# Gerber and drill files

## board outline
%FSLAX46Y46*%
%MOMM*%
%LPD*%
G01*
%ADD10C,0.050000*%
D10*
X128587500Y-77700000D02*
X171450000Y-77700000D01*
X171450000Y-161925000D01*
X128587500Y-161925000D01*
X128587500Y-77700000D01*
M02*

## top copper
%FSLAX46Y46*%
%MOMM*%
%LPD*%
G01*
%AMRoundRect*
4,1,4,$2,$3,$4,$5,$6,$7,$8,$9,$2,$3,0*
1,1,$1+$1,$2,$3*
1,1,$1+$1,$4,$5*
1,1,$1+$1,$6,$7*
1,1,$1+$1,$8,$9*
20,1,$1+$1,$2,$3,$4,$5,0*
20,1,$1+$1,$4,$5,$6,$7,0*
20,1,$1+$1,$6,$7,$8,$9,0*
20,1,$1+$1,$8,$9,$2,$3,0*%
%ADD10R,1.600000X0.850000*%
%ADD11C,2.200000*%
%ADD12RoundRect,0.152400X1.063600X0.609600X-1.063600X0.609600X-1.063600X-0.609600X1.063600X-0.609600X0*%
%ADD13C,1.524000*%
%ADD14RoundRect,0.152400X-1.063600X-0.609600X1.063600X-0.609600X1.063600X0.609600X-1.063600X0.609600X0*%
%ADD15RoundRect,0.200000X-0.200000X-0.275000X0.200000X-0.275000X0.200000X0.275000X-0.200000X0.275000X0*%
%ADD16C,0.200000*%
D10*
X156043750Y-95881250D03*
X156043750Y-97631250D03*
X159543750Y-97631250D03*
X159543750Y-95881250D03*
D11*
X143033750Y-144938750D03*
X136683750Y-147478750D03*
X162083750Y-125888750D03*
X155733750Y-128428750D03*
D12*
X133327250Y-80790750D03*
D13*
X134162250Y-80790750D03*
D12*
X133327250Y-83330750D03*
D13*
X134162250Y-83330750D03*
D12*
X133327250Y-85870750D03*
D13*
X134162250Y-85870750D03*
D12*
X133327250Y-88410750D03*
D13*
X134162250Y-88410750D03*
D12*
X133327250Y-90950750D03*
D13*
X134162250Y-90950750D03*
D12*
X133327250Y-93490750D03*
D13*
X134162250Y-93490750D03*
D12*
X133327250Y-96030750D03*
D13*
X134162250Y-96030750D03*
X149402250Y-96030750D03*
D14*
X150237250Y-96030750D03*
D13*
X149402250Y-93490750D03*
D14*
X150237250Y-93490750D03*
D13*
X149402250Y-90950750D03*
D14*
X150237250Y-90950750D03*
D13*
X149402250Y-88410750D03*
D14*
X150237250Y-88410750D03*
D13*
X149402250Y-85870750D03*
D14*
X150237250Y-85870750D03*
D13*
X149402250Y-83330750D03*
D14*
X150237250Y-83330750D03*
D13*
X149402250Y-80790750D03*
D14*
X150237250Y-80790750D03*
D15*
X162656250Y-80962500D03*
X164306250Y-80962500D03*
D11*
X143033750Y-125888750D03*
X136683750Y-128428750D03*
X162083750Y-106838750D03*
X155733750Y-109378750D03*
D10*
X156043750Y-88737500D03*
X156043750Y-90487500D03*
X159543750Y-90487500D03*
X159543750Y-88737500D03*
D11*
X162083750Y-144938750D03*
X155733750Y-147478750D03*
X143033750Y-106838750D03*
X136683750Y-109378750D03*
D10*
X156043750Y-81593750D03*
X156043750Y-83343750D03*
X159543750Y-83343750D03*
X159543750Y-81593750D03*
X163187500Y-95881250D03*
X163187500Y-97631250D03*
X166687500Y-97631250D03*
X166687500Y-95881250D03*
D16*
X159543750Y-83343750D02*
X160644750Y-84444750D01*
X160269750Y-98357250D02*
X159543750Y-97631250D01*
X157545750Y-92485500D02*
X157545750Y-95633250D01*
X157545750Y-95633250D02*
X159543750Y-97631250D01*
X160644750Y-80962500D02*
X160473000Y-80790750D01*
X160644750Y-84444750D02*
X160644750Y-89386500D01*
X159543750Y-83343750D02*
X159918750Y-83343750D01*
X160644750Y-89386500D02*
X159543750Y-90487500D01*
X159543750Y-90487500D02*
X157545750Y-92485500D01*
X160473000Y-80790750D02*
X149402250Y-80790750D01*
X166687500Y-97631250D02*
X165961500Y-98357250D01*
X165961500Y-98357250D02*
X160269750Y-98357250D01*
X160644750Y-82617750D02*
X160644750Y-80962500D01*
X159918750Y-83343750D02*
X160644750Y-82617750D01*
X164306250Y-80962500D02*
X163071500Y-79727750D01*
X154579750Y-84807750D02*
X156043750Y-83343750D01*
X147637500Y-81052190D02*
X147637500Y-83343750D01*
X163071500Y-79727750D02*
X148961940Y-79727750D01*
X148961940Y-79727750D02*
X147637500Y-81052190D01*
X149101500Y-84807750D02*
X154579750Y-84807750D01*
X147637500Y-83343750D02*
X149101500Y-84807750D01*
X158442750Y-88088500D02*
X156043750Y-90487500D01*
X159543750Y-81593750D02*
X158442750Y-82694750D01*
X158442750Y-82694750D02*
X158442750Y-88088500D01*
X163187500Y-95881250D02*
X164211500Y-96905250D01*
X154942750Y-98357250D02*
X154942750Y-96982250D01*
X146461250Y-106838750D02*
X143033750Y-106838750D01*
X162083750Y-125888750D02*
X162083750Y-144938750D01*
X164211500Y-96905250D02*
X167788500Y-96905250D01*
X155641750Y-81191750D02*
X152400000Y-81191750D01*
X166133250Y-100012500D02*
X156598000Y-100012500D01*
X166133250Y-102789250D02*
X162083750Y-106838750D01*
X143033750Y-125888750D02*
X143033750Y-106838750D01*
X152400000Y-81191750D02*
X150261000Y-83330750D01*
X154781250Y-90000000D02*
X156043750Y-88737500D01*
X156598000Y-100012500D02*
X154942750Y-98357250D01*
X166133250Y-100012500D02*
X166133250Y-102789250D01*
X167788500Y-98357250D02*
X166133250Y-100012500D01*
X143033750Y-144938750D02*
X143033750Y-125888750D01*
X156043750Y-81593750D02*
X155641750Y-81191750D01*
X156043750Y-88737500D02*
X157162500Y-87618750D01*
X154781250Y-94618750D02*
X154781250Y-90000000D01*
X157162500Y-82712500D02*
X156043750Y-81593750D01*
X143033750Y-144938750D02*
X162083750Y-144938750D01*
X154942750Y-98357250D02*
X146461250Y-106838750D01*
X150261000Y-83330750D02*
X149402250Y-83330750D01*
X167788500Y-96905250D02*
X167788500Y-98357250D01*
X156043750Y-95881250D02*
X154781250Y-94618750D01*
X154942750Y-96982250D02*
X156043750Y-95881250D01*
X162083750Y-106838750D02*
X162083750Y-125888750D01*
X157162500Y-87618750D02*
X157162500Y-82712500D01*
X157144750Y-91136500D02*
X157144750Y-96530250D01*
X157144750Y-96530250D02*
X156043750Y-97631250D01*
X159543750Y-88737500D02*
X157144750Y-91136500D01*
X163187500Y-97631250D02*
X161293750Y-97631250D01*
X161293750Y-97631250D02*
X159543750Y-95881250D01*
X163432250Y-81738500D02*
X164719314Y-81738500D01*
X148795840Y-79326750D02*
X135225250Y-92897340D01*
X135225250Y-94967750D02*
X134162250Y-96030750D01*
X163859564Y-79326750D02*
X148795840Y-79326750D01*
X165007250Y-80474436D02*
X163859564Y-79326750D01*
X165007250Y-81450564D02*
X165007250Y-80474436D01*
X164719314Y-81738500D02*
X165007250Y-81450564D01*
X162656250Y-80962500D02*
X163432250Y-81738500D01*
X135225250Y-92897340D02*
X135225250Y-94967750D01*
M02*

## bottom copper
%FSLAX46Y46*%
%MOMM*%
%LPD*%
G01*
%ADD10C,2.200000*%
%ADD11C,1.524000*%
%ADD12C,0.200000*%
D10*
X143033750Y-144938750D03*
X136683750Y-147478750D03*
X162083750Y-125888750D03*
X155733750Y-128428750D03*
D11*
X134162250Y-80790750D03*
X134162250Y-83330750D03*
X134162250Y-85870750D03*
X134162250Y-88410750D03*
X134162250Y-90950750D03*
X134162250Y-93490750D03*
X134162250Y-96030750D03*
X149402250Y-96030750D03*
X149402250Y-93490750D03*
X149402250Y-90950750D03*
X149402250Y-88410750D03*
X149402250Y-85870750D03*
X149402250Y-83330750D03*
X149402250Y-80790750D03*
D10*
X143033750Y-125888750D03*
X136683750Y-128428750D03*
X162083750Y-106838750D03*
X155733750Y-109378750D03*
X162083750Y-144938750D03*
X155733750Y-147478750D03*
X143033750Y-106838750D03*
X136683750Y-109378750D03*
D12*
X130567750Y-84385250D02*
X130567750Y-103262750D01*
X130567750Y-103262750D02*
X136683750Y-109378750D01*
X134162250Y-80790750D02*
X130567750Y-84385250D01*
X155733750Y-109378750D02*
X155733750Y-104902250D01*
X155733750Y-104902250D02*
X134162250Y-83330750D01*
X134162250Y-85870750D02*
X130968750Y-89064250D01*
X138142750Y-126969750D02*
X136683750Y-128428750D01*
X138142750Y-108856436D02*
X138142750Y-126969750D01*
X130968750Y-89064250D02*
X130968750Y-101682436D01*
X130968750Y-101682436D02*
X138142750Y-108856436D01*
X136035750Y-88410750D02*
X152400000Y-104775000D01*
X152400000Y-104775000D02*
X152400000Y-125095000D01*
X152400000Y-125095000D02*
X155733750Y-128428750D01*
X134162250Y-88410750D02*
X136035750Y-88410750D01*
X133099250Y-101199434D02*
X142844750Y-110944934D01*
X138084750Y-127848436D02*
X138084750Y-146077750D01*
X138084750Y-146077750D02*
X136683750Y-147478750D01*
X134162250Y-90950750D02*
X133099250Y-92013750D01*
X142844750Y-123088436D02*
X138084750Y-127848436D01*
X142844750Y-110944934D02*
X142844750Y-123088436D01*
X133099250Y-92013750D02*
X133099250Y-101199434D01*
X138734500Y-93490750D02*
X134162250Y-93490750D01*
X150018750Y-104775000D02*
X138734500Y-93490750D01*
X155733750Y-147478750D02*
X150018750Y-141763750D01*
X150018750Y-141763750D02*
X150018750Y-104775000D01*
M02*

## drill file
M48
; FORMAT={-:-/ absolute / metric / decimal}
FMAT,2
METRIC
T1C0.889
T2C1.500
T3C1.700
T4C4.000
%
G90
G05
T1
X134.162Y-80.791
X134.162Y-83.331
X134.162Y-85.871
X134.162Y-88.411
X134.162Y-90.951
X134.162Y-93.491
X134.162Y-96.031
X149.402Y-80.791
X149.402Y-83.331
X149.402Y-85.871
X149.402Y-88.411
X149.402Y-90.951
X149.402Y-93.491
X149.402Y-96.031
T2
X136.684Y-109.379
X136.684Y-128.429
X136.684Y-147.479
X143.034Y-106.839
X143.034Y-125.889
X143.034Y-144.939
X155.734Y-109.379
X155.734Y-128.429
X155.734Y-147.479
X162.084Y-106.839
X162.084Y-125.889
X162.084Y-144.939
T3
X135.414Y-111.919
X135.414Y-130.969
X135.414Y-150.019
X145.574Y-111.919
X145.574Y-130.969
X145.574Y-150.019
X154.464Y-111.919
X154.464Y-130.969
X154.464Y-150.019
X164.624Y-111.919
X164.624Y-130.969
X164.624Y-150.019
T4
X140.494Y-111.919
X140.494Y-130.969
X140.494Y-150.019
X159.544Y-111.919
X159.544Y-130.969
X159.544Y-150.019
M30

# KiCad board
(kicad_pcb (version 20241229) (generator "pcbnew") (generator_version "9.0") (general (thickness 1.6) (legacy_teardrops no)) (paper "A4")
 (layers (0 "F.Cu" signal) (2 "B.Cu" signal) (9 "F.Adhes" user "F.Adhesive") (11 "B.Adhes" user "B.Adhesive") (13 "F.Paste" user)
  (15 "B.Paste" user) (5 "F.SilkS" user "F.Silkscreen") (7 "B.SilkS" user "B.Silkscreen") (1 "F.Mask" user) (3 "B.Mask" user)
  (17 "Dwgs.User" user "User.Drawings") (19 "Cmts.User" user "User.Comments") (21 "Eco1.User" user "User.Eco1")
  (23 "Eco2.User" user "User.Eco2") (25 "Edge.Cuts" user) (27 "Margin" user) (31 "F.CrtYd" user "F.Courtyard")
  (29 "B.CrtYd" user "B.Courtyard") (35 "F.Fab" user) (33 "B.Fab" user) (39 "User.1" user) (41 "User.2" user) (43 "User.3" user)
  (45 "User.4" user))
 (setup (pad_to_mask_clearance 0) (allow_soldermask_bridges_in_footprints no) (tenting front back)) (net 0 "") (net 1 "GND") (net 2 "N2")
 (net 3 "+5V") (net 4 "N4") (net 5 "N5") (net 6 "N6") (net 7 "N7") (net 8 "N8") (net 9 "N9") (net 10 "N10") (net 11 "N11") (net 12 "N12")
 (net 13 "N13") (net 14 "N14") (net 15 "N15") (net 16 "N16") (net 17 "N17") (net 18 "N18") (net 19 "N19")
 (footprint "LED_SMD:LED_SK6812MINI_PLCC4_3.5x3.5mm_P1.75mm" (layer "F.Cu") (at 157.79375 96.75625)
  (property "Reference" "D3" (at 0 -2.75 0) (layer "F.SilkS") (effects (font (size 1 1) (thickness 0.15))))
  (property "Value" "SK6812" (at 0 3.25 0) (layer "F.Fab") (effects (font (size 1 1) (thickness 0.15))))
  (pad "1" smd rect (at -1.75 -0.875) (size 1.6 0.85) (layers "F.Cu" "F.Mask" "F.Paste") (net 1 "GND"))
  (pad "2" smd rect (at -1.75 0.875) (size 1.6 0.85) (layers "F.Cu" "F.Mask" "F.Paste") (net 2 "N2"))
  (pad "3" smd rect (at 1.75 0.875) (size 1.6 0.85) (layers "F.Cu" "F.Mask" "F.Paste") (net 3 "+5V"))
  (pad "4" smd rect (at 1.75 -0.875) (size 1.6 0.85) (layers "F.Cu" "F.Mask" "F.Paste") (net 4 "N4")))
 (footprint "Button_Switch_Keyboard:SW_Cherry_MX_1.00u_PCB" (layer "F.Cu") (at 143.03375 144.93875)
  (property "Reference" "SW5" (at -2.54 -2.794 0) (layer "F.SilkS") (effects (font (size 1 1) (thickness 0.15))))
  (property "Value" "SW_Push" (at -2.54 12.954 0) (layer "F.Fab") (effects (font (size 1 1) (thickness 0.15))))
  (pad "" np_thru_hole circle (at -7.62 5.08) (size 1.7 1.7) (drill 1.7) (layers "*.Cu" "*.Mask"))
  (pad "" np_thru_hole circle (at -2.54 5.08) (size 4 4) (drill 4) (layers "*.Cu" "*.Mask"))
  (pad "" np_thru_hole circle (at 2.54 5.08) (size 1.7 1.7) (drill 1.7) (layers "*.Cu" "*.Mask"))
  (pad "1" thru_hole circle (at 0 0) (size 2.2 2.2) (drill 1.5) (layers "*.Cu" "*.Mask") (remove_unused_layers no) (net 1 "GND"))
  (pad "2" thru_hole circle (at -6.35 2.54) (size 2.2 2.2) (drill 1.5) (layers "*.Cu" "*.Mask") (remove_unused_layers no) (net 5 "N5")))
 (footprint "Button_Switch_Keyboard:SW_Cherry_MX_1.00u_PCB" (layer "F.Cu") (at 162.08375 125.88875)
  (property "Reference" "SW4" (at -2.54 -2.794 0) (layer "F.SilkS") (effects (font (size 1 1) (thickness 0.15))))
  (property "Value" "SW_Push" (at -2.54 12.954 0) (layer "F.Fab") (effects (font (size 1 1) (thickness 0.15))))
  (pad "" np_thru_hole circle (at -7.62 5.08) (size 1.7 1.7) (drill 1.7) (layers "*.Cu" "*.Mask"))
  (pad "" np_thru_hole circle (at -2.54 5.08) (size 4 4) (drill 4) (layers "*.Cu" "*.Mask"))
  (pad "" np_thru_hole circle (at 2.54 5.08) (size 1.7 1.7) (drill 1.7) (layers "*.Cu" "*.Mask"))
  (pad "1" thru_hole circle (at 0 0) (size 2.2 2.2) (drill 1.5) (layers "*.Cu" "*.Mask") (remove_unused_layers no) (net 1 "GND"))
  (pad "2" thru_hole circle (at -6.35 2.54) (size 2.2 2.2) (drill 1.5) (layers "*.Cu" "*.Mask") (remove_unused_layers no) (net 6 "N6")))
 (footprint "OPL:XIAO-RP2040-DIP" (layer "F.Cu") (at 141.78225 88.41075)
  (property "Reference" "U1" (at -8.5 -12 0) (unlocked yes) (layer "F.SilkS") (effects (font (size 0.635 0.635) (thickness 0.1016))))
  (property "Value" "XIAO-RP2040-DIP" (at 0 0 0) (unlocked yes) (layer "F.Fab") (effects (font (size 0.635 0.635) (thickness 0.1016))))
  (pad "1" smd roundrect (at -8.455 -7.62 180) (size 2.432 1.524) (layers "F.Cu" "F.Mask") (roundrect_rratio 0.1) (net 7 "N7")
   (thermal_bridge_angle 45))
  (pad "1" thru_hole circle (at -7.62 -7.62 180) (size 1.524 1.524) (drill 0.889) (layers "*.Cu" "*.Mask") (remove_unused_layers no)
   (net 7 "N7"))
  (pad "2" smd roundrect (at -8.455 -5.08 180) (size 2.432 1.524) (layers "F.Cu" "F.Mask") (roundrect_rratio 0.1) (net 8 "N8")
   (thermal_bridge_angle 45))
  (pad "2" thru_hole circle (at -7.62 -5.08 180) (size 1.524 1.524) (drill 0.889) (layers "*.Cu" "*.Mask") (remove_unused_layers no)
   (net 8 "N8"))
  (pad "3" smd roundrect (at -8.455 -2.54 180) (size 2.432 1.524) (layers "F.Cu" "F.Mask") (roundrect_rratio 0.1) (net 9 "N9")
   (thermal_bridge_angle 45))
  (pad "3" thru_hole circle (at -7.62 -2.54 180) (size 1.524 1.524) (drill 0.889) (layers "*.Cu" "*.Mask") (remove_unused_layers no)
   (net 9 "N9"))
  (pad "4" smd roundrect (at -8.455 0 180) (size 2.432 1.524) (layers "F.Cu" "F.Mask") (roundrect_rratio 0.1) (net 6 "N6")
   (thermal_bridge_angle 45))
  (pad "4" thru_hole circle (at -7.62 0 180) (size 1.524 1.524) (drill 0.889) (layers "*.Cu" "*.Mask") (remove_unused_layers no)
   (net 6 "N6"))
  (pad "5" smd roundrect (at -8.455 2.54 180) (size 2.432 1.524) (layers "F.Cu" "F.Mask") (roundrect_rratio 0.1) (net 5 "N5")
   (thermal_bridge_angle 45))
  (pad "5" thru_hole circle (at -7.62 2.54 180) (size 1.524 1.524) (drill 0.889) (layers "*.Cu" "*.Mask") (remove_unused_layers no)
   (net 5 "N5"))
  (pad "6" smd roundrect (at -8.455 5.08 180) (size 2.432 1.524) (layers "F.Cu" "F.Mask") (roundrect_rratio 0.1) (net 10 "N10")
   (thermal_bridge_angle 45))
  (pad "6" thru_hole circle (at -7.62 5.08 180) (size 1.524 1.524) (drill 0.889) (layers "*.Cu" "*.Mask") (remove_unused_layers no)
   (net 10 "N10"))
  (pad "7" smd roundrect (at -8.455 7.62 180) (size 2.432 1.524) (layers "F.Cu" "F.Mask") (roundrect_rratio 0.1) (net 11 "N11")
   (thermal_bridge_angle 45))
  (pad "7" thru_hole circle (at -7.62 7.62 180) (size 1.524 1.524) (drill 0.889) (layers "*.Cu" "*.Mask") (remove_unused_layers no)
   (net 11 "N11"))
  (pad "8" thru_hole circle (at 7.62 7.62) (size 1.524 1.524) (drill 0.889) (layers "*.Cu" "*.Mask") (remove_unused_layers no)
   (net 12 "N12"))
  (pad "8" smd roundrect (at 8.455 7.62) (size 2.432 1.524) (layers "F.Cu" "F.Mask") (roundrect_rratio 0.1) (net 12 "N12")
   (thermal_bridge_angle 45))
  (pad "9" thru_hole circle (at 7.62 5.08) (size 1.524 1.524) (drill 0.889) (layers "*.Cu" "*.Mask") (remove_unused_layers no)
   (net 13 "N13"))
  (pad "9" smd roundrect (at 8.455 5.08) (size 2.432 1.524) (layers "F.Cu" "F.Mask") (roundrect_rratio 0.1) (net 13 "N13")
   (thermal_bridge_angle 45))
  (pad "10" thru_hole circle (at 7.62 2.54) (size 1.524 1.524) (drill 0.889) (layers "*.Cu" "*.Mask") (remove_unused_layers no)
   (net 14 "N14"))
  (pad "10" smd roundrect (at 8.455 2.54) (size 2.432 1.524) (layers "F.Cu" "F.Mask") (roundrect_rratio 0.1) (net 14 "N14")
   (thermal_bridge_angle 45))
  (pad "11" thru_hole circle (at 7.62 0) (size 1.524 1.524) (drill 0.889) (layers "*.Cu" "*.Mask") (remove_unused_layers no) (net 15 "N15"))
  (pad "11" smd roundrect (at 8.455 0) (size 2.432 1.524) (layers "F.Cu" "F.Mask") (roundrect_rratio 0.1) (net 15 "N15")
   (thermal_bridge_angle 45))
  (pad "12" thru_hole circle (at 7.62 -2.54) (size 1.524 1.524) (drill 0.889) (layers "*.Cu" "*.Mask") (remove_unused_layers no)
   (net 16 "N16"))
  (pad "12" smd roundrect (at 8.455 -2.54) (size 2.432 1.524) (layers "F.Cu" "F.Mask") (roundrect_rratio 0.1) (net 16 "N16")
   (thermal_bridge_angle 45))
  (pad "13" thru_hole circle (at 7.62 -5.08) (size 1.524 1.524) (drill 0.889) (layers "*.Cu" "*.Mask") (remove_unused_layers no)
   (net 1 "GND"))
  (pad "13" smd roundrect (at 8.455 -5.08) (size 2.432 1.524) (layers "F.Cu" "F.Mask") (roundrect_rratio 0.1) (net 1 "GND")
   (thermal_bridge_angle 45))
  (pad "14" thru_hole circle (at 7.62 -7.62) (size 1.524 1.524) (drill 0.889) (layers "*.Cu" "*.Mask") (remove_unused_layers no)
   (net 3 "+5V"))
  (pad "14" smd roundrect (at 8.455 -7.62) (size 2.432 1.524) (layers "F.Cu" "F.Mask") (roundrect_rratio 0.1) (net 3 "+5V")
   (thermal_bridge_angle 45)))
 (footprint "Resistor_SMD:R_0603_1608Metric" (layer "F.Cu") (at 163.48125 80.9625)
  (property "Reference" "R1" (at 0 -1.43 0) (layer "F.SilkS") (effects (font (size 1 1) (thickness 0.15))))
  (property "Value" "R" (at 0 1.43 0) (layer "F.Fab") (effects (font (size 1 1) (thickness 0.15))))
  (pad "1" smd roundrect (at -0.825 0) (size 0.8 0.95) (layers "F.Cu" "F.Mask" "F.Paste") (roundrect_rratio 0.25) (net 11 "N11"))
  (pad "2" smd roundrect (at 0.825 0) (size 0.8 0.95) (layers "F.Cu" "F.Mask" "F.Paste") (roundrect_rratio 0.25) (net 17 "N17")))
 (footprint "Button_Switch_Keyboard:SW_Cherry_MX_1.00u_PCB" (layer "F.Cu") (at 143.03375 125.88875)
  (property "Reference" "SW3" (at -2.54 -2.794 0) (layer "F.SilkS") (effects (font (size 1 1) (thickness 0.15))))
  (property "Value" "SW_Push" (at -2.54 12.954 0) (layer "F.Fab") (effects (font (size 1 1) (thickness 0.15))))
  (pad "" np_thru_hole circle (at -7.62 5.08) (size 1.7 1.7) (drill 1.7) (layers "*.Cu" "*.Mask"))
  (pad "" np_thru_hole circle (at -2.54 5.08) (size 4 4) (drill 4) (layers "*.Cu" "*.Mask"))
  (pad "" np_thru_hole circle (at 2.54 5.08) (size 1.7 1.7) (drill 1.7) (layers "*.Cu" "*.Mask"))
  (pad "1" thru_hole circle (at 0 0) (size 2.2 2.2) (drill 1.5) (layers "*.Cu" "*.Mask") (remove_unused_layers no) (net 1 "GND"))
  (pad "2" thru_hole circle (at -6.35 2.54) (size 2.2 2.2) (drill 1.5) (layers "*.Cu" "*.Mask") (remove_unused_layers no) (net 9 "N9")))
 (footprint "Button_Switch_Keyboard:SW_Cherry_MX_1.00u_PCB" (layer "F.Cu") (at 162.08375 106.83875)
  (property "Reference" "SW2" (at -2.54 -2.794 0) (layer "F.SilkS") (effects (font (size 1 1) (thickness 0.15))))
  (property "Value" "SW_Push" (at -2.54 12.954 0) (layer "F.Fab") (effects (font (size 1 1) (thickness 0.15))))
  (pad "" np_thru_hole circle (at -7.62 5.08) (size 1.7 1.7) (drill 1.7) (layers "*.Cu" "*.Mask"))
  (pad "" np_thru_hole circle (at -2.54 5.08) (size 4 4) (drill 4) (layers "*.Cu" "*.Mask"))
  (pad "" np_thru_hole circle (at 2.54 5.08) (size 1.7 1.7) (drill 1.7) (layers "*.Cu" "*.Mask"))
  (pad "1" thru_hole circle (at 0 0) (size 2.2 2.2) (drill 1.5) (layers "*.Cu" "*.Mask") (remove_unused_layers no) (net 1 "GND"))
  (pad "2" thru_hole circle (at -6.35 2.54) (size 2.2 2.2) (drill 1.5) (layers "*.Cu" "*.Mask") (remove_unused_layers no) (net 8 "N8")))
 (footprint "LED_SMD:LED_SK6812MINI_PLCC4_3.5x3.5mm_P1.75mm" (layer "F.Cu") (at 157.79375 89.6125)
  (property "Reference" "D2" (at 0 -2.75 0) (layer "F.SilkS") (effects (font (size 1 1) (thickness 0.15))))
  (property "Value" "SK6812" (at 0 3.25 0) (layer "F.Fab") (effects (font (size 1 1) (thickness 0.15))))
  (pad "1" smd rect (at -1.75 -0.875) (size 1.6 0.85) (layers "F.Cu" "F.Mask" "F.Paste") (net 1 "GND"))
  (pad "2" smd rect (at -1.75 0.875) (size 1.6 0.85) (layers "F.Cu" "F.Mask" "F.Paste") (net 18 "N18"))
  (pad "3" smd rect (at 1.75 0.875) (size 1.6 0.85) (layers "F.Cu" "F.Mask" "F.Paste") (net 3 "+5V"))
  (pad "4" smd rect (at 1.75 -0.875) (size 1.6 0.85) (layers "F.Cu" "F.Mask" "F.Paste") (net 2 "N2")))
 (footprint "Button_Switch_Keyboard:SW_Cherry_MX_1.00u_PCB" (layer "F.Cu") (at 162.08375 144.93875)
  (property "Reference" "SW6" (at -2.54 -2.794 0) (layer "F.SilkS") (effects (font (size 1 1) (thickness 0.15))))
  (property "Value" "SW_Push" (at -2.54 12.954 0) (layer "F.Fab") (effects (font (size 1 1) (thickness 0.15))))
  (pad "" np_thru_hole circle (at -7.62 5.08) (size 1.7 1.7) (drill 1.7) (layers "*.Cu" "*.Mask"))
  (pad "" np_thru_hole circle (at -2.54 5.08) (size 4 4) (drill 4) (layers "*.Cu" "*.Mask"))
  (pad "" np_thru_hole circle (at 2.54 5.08) (size 1.7 1.7) (drill 1.7) (layers "*.Cu" "*.Mask"))
  (pad "1" thru_hole circle (at 0 0) (size 2.2 2.2) (drill 1.5) (layers "*.Cu" "*.Mask") (remove_unused_layers no) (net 1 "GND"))
  (pad "2" thru_hole circle (at -6.35 2.54) (size 2.2 2.2) (drill 1.5) (layers "*.Cu" "*.Mask") (remove_unused_layers no) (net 10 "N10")))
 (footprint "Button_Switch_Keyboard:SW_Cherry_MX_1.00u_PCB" (layer "F.Cu") (at 143.03375 106.83875)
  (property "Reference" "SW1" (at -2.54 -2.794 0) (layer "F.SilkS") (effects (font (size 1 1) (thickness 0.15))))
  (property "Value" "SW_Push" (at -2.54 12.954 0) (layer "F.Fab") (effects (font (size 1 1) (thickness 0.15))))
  (pad "" np_thru_hole circle (at -7.62 5.08) (size 1.7 1.7) (drill 1.7) (layers "*.Cu" "*.Mask"))
  (pad "" np_thru_hole circle (at -2.54 5.08) (size 4 4) (drill 4) (layers "*.Cu" "*.Mask"))
  (pad "" np_thru_hole circle (at 2.54 5.08) (size 1.7 1.7) (drill 1.7) (layers "*.Cu" "*.Mask"))
  (pad "1" thru_hole circle (at 0 0) (size 2.2 2.2) (drill 1.5) (layers "*.Cu" "*.Mask") (remove_unused_layers no) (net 1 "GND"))
  (pad "2" thru_hole circle (at -6.35 2.54) (size 2.2 2.2) (drill 1.5) (layers "*.Cu" "*.Mask") (remove_unused_layers no) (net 7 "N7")))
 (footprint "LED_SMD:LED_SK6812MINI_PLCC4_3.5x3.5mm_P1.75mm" (layer "F.Cu") (at 157.79375 82.46875)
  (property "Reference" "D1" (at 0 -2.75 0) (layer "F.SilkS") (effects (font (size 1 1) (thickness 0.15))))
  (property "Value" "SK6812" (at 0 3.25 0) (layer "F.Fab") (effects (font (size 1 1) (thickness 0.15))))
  (pad "1" smd rect (at -1.75 -0.875) (size 1.6 0.85) (layers "F.Cu" "F.Mask" "F.Paste") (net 1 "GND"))
  (pad "2" smd rect (at -1.75 0.875) (size 1.6 0.85) (layers "F.Cu" "F.Mask" "F.Paste") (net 17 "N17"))
  (pad "3" smd rect (at 1.75 0.875) (size 1.6 0.85) (layers "F.Cu" "F.Mask" "F.Paste") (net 3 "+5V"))
  (pad "4" smd rect (at 1.75 -0.875) (size 1.6 0.85) (layers "F.Cu" "F.Mask" "F.Paste") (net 18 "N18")))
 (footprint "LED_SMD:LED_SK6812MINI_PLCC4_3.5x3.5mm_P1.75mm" (layer "F.Cu") (at 164.9375 96.75625)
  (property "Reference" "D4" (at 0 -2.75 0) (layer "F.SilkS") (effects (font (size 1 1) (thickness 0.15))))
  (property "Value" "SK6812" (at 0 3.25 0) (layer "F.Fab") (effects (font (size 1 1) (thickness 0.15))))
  (pad "1" smd rect (at -1.75 -0.875) (size 1.6 0.85) (layers "F.Cu" "F.Mask" "F.Paste") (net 1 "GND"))
  (pad "2" smd rect (at -1.75 0.875) (size 1.6 0.85) (layers "F.Cu" "F.Mask" "F.Paste") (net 4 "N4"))
  (pad "3" smd rect (at 1.75 0.875) (size 1.6 0.85) (layers "F.Cu" "F.Mask" "F.Paste") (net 3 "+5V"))
  (pad "4" smd rect (at 1.75 -0.875) (size 1.6 0.85) (layers "F.Cu" "F.Mask" "F.Paste") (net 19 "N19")))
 (gr_rect (start 128.5875 77.7) (end 171.45 161.925) (stroke (width 0.05) (type solid)) (fill no) (layer "Edge.Cuts"))
 (segment (start 159.54375 83.34375) (end 160.64475 84.44475) (width 0.2) (layer "F.Cu") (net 3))
 (segment (start 160.26975 98.35725) (end 159.54375 97.63125) (width 0.2) (layer "F.Cu") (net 3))
 (segment (start 157.54575 92.4855) (end 157.54575 95.63325) (width 0.2) (layer "F.Cu") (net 3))
 (segment (start 157.54575 95.63325) (end 159.54375 97.63125) (width 0.2) (layer "F.Cu") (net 3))
 (segment (start 160.64475 80.9625) (end 160.473 80.79075) (width 0.2) (layer "F.Cu") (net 3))
 (segment (start 160.64475 84.44475) (end 160.64475 89.3865) (width 0.2) (layer "F.Cu") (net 3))
 (segment (start 159.54375 83.34375) (end 159.91875 83.34375) (width 0.2) (layer "F.Cu") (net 3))
 (segment (start 160.64475 89.3865) (end 159.54375 90.4875) (width 0.2) (layer "F.Cu") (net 3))
 (segment (start 159.54375 90.4875) (end 157.54575 92.4855) (width 0.2) (layer "F.Cu") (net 3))
 (segment (start 160.473 80.79075) (end 149.40225 80.79075) (width 0.2) (layer "F.Cu") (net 3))
 (segment (start 166.6875 97.63125) (end 165.9615 98.35725) (width 0.2) (layer "F.Cu") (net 3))
 (segment (start 165.9615 98.35725) (end 160.26975 98.35725) (width 0.2) (layer "F.Cu") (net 3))
 (segment (start 160.64475 82.61775) (end 160.64475 80.9625) (width 0.2) (layer "F.Cu") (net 3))
 (segment (start 159.91875 83.34375) (end 160.64475 82.61775) (width 0.2) (layer "F.Cu") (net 3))
 (segment (start 164.30625 80.9625) (end 163.0715 79.72775) (width 0.2) (layer "F.Cu") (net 17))
 (segment (start 154.57975 84.80775) (end 156.04375 83.34375) (width 0.2) (layer "F.Cu") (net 17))
 (segment (start 147.6375 81.05219) (end 147.6375 83.34375) (width 0.2) (layer "F.Cu") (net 17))
 (segment (start 163.0715 79.72775) (end 148.96194 79.72775) (width 0.2) (layer "F.Cu") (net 17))
 (segment (start 148.96194 79.72775) (end 147.6375 81.05219) (width 0.2) (layer "F.Cu") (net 17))
 (segment (start 149.1015 84.80775) (end 154.57975 84.80775) (width 0.2) (layer "F.Cu") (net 17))
 (segment (start 147.6375 83.34375) (end 149.1015 84.80775) (width 0.2) (layer "F.Cu") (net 17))
 (segment (start 158.44275 88.0885) (end 156.04375 90.4875) (width 0.2) (layer "F.Cu") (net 18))
 (segment (start 159.54375 81.59375) (end 158.44275 82.69475) (width 0.2) (layer "F.Cu") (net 18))
 (segment (start 158.44275 82.69475) (end 158.44275 88.0885) (width 0.2) (layer "F.Cu") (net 18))
 (segment (start 163.1875 95.88125) (end 164.2115 96.90525) (width 0.2) (layer "F.Cu") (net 1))
 (segment (start 154.94275 98.35725) (end 154.94275 96.98225) (width 0.2) (layer "F.Cu") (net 1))
 (segment (start 146.46125 106.83875) (end 143.03375 106.83875) (width 0.2) (layer "F.Cu") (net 1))
 (segment (start 162.08375 125.88875) (end 162.08375 144.93875) (width 0.2) (layer "F.Cu") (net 1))
 (segment (start 164.2115 96.90525) (end 167.7885 96.90525) (width 0.2) (layer "F.Cu") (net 1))
 (segment (start 155.64175 81.19175) (end 152.4 81.19175) (width 0.2) (layer "F.Cu") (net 1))
 (segment (start 166.13325 100.0125) (end 156.598 100.0125) (width 0.2) (layer "F.Cu") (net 1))
 (segment (start 166.13325 102.78925) (end 162.08375 106.83875) (width 0.2) (layer "F.Cu") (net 1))
 (segment (start 143.03375 125.88875) (end 143.03375 106.83875) (width 0.2) (layer "F.Cu") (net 1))
 (segment (start 152.4 81.19175) (end 150.261 83.33075) (width 0.2) (layer "F.Cu") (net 1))
 (segment (start 154.78125 90) (end 156.04375 88.7375) (width 0.2) (layer "F.Cu") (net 1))
 (segment (start 156.598 100.0125) (end 154.94275 98.35725) (width 0.2) (layer "F.Cu") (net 1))
 (segment (start 166.13325 100.0125) (end 166.13325 102.78925) (width 0.2) (layer "F.Cu") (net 1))
 (segment (start 167.7885 98.35725) (end 166.13325 100.0125) (width 0.2) (layer "F.Cu") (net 1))
 (segment (start 143.03375 144.93875) (end 143.03375 125.88875) (width 0.2) (layer "F.Cu") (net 1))
 (segment (start 156.04375 81.59375) (end 155.64175 81.19175) (width 0.2) (layer "F.Cu") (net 1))
 (segment (start 156.04375 88.7375) (end 157.1625 87.61875) (width 0.2) (layer "F.Cu") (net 1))
 (segment (start 154.78125 94.61875) (end 154.78125 90) (width 0.2) (layer "F.Cu") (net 1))
 (segment (start 157.1625 82.7125) (end 156.04375 81.59375) (width 0.2) (layer "F.Cu") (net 1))
 (segment (start 143.03375 144.93875) (end 162.08375 144.93875) (width 0.2) (layer "F.Cu") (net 1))
 (segment (start 154.94275 98.35725) (end 146.46125 106.83875) (width 0.2) (layer "F.Cu") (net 1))
 (segment (start 150.261 83.33075) (end 149.40225 83.33075) (width 0.2) (layer "F.Cu") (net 1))
 (segment (start 167.7885 96.90525) (end 167.7885 98.35725) (width 0.2) (layer "F.Cu") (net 1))
 (segment (start 156.04375 95.88125) (end 154.78125 94.61875) (width 0.2) (layer "F.Cu") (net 1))
 (segment (start 154.94275 96.98225) (end 156.04375 95.88125) (width 0.2) (layer "F.Cu") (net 1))
 (segment (start 162.08375 106.83875) (end 162.08375 125.88875) (width 0.2) (layer "F.Cu") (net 1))
 (segment (start 157.1625 87.61875) (end 157.1625 82.7125) (width 0.2) (layer "F.Cu") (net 1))
 (segment (start 157.14475 91.1365) (end 157.14475 96.53025) (width 0.2) (layer "F.Cu") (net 2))
 (segment (start 157.14475 96.53025) (end 156.04375 97.63125) (width 0.2) (layer "F.Cu") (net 2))
 (segment (start 159.54375 88.7375) (end 157.14475 91.1365) (width 0.2) (layer "F.Cu") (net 2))
 (segment (start 163.1875 97.63125) (end 161.29375 97.63125) (width 0.2) (layer "F.Cu") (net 4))
 (segment (start 161.29375 97.63125) (end 159.54375 95.88125) (width 0.2) (layer "F.Cu") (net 4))
 (segment (start 163.43225 81.7385) (end 164.719314 81.7385) (width 0.2) (layer "F.Cu") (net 11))
 (segment (start 148.79584 79.32675) (end 135.22525 92.89734) (width 0.2) (layer "F.Cu") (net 11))
 (segment (start 135.22525 94.96775) (end 134.16225 96.03075) (width 0.2) (layer "F.Cu") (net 11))
 (segment (start 163.859564 79.32675) (end 148.79584 79.32675) (width 0.2) (layer "F.Cu") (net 11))
 (segment (start 165.00725 80.474436) (end 163.859564 79.32675) (width 0.2) (layer "F.Cu") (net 11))
 (segment (start 165.00725 81.450564) (end 165.00725 80.474436) (width 0.2) (layer "F.Cu") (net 11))
 (segment (start 164.719314 81.7385) (end 165.00725 81.450564) (width 0.2) (layer "F.Cu") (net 11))
 (segment (start 162.65625 80.9625) (end 163.43225 81.7385) (width 0.2) (layer "F.Cu") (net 11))
 (segment (start 135.22525 92.89734) (end 135.22525 94.96775) (width 0.2) (layer "F.Cu") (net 11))
 (segment (start 130.56775 84.38525) (end 130.56775 103.26275) (width 0.2) (layer "B.Cu") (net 7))
 (segment (start 130.56775 103.26275) (end 136.68375 109.37875) (width 0.2) (layer "B.Cu") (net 7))
 (segment (start 134.16225 80.79075) (end 130.56775 84.38525) (width 0.2) (layer "B.Cu") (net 7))
 (segment (start 155.73375 109.37875) (end 155.73375 104.90225) (width 0.2) (layer "B.Cu") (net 8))
 (segment (start 155.73375 104.90225) (end 134.16225 83.33075) (width 0.2) (layer "B.Cu") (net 8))
 (segment (start 134.16225 85.87075) (end 130.96875 89.06425) (width 0.2) (layer "B.Cu") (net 9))
 (segment (start 138.14275 126.96975) (end 136.68375 128.42875) (width 0.2) (layer "B.Cu") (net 9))
 (segment (start 138.14275 108.856436) (end 138.14275 126.96975) (width 0.2) (layer "B.Cu") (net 9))
 (segment (start 130.96875 89.06425) (end 130.96875 101.682436) (width 0.2) (layer "B.Cu") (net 9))
 (segment (start 130.96875 101.682436) (end 138.14275 108.856436) (width 0.2) (layer "B.Cu") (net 9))
 (segment (start 136.03575 88.41075) (end 152.4 104.775) (width 0.2) (layer "B.Cu") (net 6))
 (segment (start 152.4 104.775) (end 152.4 125.095) (width 0.2) (layer "B.Cu") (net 6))
 (segment (start 152.4 125.095) (end 155.73375 128.42875) (width 0.2) (layer "B.Cu") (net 6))
 (segment (start 134.16225 88.41075) (end 136.03575 88.41075) (width 0.2) (layer "B.Cu") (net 6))
 (segment (start 133.09925 101.199434) (end 142.84475 110.944934) (width 0.2) (layer "B.Cu") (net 5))
 (segment (start 138.08475 127.848436) (end 138.08475 146.07775) (width 0.2) (layer "B.Cu") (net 5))
 (segment (start 138.08475 146.07775) (end 136.68375 147.47875) (width 0.2) (layer "B.Cu") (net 5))
 (segment (start 134.16225 90.95075) (end 133.09925 92.01375) (width 0.2) (layer "B.Cu") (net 5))
 (segment (start 142.84475 123.088436) (end 138.08475 127.848436) (width 0.2) (layer "B.Cu") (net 5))
 (segment (start 142.84475 110.944934) (end 142.84475 123.088436) (width 0.2) (layer "B.Cu") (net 5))
 (segment (start 133.09925 92.01375) (end 133.09925 101.199434) (width 0.2) (layer "B.Cu") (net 5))
 (segment (start 138.7345 93.49075) (end 134.16225 93.49075) (width 0.2) (layer "B.Cu") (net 10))
 (segment (start 150.01875 104.775) (end 138.7345 93.49075) (width 0.2) (layer "B.Cu") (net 10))
 (segment (start 155.73375 147.47875) (end 150.01875 141.76375) (width 0.2) (layer "B.Cu") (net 10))
 (segment (start 150.01875 141.76375) (end 150.01875 104.775) (width 0.2) (layer "B.Cu") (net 10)))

